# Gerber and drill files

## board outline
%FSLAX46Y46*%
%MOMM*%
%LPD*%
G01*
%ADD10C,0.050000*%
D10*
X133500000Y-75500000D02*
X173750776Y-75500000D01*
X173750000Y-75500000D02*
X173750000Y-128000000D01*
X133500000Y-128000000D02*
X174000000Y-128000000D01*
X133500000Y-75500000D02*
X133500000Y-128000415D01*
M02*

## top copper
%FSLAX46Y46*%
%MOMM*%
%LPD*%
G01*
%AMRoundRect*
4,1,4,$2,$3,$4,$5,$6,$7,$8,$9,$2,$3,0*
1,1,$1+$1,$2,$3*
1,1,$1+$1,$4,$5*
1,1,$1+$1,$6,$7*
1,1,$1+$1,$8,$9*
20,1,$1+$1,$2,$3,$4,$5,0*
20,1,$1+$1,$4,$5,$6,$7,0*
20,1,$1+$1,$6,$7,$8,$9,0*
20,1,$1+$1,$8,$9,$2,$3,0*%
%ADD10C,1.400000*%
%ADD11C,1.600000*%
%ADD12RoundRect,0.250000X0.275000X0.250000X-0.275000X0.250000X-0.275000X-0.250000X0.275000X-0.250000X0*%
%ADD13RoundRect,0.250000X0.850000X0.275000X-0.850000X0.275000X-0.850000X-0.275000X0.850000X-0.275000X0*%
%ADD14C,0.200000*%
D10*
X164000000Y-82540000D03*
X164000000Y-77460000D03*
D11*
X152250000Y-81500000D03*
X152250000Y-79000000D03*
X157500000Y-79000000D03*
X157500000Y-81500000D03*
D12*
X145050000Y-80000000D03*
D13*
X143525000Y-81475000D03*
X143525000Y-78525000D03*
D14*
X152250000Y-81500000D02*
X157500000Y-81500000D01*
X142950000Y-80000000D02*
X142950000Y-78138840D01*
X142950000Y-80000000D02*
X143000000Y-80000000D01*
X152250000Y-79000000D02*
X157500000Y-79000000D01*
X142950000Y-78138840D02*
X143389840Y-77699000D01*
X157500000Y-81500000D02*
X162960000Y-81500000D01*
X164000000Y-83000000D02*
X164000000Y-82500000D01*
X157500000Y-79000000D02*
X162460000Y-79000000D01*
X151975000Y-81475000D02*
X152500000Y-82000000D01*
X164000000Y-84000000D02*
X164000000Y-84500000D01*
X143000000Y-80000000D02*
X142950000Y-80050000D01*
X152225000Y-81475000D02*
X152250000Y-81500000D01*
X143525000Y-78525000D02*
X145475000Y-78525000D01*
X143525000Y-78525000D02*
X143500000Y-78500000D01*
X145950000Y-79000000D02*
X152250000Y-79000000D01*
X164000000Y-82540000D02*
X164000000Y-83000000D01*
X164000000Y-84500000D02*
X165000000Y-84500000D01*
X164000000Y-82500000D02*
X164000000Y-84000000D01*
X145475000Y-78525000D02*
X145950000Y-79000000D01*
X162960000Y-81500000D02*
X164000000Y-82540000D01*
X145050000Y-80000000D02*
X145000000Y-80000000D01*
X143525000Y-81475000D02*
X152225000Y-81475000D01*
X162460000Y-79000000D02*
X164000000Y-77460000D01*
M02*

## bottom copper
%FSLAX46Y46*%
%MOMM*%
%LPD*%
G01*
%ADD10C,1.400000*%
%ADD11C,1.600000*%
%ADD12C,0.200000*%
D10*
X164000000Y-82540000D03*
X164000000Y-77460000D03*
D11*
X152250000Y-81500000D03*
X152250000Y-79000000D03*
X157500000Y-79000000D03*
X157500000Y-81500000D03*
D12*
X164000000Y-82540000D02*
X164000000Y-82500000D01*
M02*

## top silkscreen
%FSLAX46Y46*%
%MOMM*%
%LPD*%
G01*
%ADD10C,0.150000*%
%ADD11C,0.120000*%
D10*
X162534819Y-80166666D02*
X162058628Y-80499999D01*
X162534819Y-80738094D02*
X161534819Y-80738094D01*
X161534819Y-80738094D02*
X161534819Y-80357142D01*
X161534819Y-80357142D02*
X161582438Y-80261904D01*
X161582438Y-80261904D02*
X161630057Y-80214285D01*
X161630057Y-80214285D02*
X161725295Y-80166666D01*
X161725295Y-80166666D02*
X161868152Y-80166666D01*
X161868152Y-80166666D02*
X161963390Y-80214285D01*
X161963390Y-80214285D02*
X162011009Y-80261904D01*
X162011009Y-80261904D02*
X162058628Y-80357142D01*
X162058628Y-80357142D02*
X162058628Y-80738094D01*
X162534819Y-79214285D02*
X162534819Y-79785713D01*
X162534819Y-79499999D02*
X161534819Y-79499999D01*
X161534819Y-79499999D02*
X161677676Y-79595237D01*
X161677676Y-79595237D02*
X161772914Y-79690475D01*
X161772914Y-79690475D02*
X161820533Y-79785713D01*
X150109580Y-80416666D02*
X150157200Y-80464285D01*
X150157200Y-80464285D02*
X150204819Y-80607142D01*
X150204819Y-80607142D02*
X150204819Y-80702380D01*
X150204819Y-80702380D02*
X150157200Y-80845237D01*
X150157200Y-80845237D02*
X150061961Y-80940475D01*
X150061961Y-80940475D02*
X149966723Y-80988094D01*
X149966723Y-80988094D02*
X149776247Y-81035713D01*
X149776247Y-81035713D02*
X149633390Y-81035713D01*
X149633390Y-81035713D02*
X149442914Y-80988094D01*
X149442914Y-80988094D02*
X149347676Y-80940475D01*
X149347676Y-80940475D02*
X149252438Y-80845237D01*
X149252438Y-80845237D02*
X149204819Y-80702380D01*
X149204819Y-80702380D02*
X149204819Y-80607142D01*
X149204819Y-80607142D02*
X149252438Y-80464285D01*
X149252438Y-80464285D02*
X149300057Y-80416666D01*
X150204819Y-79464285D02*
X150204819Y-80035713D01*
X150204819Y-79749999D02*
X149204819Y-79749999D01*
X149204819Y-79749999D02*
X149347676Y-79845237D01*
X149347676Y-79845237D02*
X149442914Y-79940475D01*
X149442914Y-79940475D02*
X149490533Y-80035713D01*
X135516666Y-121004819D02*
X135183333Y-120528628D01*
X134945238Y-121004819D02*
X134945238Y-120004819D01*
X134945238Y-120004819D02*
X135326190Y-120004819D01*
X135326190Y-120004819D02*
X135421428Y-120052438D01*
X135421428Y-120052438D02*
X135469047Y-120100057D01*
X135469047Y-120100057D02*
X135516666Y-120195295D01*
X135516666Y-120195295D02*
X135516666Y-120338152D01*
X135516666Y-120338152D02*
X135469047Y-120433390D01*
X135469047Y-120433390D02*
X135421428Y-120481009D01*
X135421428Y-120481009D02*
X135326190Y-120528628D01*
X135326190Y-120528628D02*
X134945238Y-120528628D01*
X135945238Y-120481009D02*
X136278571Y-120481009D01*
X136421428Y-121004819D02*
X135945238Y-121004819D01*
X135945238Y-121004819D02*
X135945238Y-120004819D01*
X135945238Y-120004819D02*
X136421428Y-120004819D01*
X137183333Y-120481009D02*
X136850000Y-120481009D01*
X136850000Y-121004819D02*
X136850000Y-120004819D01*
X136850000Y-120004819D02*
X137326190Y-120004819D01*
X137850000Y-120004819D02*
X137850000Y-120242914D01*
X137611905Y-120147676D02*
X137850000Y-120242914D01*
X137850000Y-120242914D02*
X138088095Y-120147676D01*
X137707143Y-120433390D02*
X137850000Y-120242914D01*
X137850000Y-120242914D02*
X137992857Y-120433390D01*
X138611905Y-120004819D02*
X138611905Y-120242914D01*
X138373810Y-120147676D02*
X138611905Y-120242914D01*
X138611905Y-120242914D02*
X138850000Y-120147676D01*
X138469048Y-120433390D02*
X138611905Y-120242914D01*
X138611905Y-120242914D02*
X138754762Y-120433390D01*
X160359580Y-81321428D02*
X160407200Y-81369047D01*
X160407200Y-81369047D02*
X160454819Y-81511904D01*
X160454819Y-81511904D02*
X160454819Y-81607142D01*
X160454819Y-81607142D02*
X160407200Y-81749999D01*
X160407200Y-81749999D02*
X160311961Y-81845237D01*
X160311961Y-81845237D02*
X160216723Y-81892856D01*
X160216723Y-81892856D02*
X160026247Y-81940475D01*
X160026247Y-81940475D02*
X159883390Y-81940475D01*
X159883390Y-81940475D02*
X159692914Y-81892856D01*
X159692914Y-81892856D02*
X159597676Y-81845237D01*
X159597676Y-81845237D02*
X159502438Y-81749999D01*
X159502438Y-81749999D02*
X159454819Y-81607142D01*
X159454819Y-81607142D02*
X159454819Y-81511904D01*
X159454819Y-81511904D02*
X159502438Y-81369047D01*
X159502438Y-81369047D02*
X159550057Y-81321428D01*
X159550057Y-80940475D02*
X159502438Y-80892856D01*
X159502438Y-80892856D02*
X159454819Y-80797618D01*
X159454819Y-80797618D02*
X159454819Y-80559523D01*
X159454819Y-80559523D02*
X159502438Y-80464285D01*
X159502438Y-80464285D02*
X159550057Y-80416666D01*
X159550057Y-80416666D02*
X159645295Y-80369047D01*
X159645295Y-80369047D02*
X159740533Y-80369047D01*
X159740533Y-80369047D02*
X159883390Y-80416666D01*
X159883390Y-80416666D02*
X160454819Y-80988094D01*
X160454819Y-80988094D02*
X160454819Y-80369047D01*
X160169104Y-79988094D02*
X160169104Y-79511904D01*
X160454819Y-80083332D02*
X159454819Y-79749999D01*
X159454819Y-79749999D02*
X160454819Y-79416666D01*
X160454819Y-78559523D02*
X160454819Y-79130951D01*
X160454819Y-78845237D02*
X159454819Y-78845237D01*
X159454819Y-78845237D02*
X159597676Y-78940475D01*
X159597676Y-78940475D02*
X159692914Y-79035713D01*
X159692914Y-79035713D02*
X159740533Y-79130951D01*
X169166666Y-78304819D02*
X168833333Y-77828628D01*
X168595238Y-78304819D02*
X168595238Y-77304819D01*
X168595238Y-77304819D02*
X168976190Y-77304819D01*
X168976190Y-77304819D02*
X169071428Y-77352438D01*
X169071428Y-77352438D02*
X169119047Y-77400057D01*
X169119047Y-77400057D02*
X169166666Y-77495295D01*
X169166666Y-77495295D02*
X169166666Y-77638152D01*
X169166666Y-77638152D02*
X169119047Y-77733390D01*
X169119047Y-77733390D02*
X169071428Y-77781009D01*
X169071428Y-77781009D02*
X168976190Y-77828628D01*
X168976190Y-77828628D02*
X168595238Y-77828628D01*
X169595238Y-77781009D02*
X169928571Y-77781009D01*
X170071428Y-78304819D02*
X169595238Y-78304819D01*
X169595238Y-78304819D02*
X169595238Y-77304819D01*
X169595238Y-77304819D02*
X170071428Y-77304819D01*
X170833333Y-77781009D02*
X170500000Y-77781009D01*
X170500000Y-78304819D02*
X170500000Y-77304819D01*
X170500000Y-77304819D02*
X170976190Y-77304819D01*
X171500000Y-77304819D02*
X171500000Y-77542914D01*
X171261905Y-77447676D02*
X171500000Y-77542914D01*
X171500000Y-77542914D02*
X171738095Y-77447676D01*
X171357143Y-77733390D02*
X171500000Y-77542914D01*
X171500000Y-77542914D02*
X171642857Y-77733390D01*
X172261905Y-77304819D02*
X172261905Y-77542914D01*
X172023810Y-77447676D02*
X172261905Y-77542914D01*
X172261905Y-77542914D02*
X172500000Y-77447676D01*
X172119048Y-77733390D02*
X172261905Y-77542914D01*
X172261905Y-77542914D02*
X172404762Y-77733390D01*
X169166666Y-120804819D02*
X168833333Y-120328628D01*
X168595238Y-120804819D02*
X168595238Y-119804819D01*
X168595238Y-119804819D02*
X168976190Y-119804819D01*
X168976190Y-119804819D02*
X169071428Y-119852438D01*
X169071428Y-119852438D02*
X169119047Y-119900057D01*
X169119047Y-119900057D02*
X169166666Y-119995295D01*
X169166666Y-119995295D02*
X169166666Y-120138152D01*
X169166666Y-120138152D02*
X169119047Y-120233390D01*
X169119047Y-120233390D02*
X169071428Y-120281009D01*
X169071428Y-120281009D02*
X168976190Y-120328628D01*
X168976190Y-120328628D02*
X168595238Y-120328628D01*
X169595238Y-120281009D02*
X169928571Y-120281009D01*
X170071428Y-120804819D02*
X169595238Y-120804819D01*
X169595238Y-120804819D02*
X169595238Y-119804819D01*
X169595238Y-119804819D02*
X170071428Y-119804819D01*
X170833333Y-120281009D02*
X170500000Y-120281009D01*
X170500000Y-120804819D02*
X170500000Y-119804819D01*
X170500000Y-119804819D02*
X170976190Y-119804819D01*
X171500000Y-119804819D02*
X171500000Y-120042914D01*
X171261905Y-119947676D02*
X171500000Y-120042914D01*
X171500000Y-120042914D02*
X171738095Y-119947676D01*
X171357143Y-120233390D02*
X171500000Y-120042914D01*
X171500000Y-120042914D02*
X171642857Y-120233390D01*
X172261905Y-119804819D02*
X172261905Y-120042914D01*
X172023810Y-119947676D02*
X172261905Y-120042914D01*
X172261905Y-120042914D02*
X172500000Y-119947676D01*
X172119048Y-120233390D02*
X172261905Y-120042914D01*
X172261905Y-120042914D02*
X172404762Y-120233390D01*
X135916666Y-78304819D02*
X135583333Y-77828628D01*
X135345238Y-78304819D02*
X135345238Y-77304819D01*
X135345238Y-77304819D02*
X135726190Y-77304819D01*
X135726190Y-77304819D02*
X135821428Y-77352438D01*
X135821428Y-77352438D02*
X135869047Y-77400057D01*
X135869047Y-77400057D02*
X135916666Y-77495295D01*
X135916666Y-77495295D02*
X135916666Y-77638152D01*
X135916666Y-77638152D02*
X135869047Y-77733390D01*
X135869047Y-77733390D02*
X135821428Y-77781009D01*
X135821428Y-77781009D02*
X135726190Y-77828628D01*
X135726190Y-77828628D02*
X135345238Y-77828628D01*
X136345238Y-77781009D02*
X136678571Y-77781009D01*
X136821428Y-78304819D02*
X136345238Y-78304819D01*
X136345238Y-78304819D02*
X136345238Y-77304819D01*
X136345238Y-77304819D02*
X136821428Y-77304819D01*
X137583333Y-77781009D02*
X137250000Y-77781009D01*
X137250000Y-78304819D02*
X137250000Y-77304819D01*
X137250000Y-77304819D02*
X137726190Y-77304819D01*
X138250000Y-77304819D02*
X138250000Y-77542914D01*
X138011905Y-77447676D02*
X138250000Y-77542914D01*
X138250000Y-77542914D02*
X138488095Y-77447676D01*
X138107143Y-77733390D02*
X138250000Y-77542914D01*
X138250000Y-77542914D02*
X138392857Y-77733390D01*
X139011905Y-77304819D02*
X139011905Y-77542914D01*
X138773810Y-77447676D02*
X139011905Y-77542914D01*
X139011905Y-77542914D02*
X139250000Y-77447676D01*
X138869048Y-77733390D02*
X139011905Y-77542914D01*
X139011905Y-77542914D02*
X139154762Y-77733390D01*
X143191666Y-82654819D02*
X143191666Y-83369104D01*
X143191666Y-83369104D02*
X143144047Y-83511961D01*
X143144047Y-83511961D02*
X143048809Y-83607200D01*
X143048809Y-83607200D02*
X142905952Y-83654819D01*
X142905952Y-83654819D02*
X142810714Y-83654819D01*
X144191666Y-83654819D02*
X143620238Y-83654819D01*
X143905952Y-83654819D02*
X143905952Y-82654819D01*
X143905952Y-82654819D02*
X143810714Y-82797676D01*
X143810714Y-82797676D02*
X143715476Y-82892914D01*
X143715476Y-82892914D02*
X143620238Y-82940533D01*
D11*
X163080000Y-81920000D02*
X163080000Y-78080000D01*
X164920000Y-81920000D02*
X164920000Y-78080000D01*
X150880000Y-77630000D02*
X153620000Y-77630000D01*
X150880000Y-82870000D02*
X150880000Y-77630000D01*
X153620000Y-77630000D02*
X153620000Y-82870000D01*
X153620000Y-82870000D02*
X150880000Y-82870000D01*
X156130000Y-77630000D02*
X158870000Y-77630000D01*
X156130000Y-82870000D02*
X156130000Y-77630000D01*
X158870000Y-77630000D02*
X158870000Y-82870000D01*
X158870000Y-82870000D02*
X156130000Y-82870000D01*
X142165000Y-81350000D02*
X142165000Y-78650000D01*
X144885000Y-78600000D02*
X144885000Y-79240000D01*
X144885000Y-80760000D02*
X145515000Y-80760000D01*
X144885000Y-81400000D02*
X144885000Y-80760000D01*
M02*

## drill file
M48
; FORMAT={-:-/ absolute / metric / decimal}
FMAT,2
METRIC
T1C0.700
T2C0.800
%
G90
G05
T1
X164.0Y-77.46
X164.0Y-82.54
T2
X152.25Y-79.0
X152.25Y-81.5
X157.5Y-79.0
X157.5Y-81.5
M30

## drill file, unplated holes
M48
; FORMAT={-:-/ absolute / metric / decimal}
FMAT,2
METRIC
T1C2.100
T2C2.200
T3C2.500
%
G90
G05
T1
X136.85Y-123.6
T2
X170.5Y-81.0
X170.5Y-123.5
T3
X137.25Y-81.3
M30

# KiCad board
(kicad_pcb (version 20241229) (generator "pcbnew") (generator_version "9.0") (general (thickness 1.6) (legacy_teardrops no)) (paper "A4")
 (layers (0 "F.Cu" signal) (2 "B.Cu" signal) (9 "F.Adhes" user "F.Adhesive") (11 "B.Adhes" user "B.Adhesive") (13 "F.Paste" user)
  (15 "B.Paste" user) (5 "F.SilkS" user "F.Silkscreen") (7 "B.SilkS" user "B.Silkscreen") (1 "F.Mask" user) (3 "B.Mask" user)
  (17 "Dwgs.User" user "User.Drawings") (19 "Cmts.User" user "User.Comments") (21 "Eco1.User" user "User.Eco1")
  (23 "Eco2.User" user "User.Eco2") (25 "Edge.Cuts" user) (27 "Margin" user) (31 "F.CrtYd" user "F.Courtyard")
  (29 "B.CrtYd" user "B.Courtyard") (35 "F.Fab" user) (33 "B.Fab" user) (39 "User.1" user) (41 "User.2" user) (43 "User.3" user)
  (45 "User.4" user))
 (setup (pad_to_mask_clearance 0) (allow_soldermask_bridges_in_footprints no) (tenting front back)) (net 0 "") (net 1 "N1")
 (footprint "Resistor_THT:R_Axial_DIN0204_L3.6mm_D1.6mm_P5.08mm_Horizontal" (layer "F.Cu") (at 164 82.54 90)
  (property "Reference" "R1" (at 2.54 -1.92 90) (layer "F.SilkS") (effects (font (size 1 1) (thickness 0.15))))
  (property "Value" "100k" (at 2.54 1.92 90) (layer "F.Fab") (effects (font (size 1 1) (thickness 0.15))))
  (fp_line (start 0.62 -0.92) (end 4.46 -0.92) (stroke (width 0.12) (type solid)) (layer "F.SilkS"))
  (fp_line (start 0.62 0.92) (end 4.46 0.92) (stroke (width 0.12) (type solid)) (layer "F.SilkS"))
  (pad "1" thru_hole circle (at 0 0 90) (size 1.4 1.4) (drill 0.7) (layers "*.Cu" "*.Mask") (remove_unused_layers no) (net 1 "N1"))
  (pad "2" thru_hole circle (at 5.08 0 90) (size 1.4 1.4) (drill 0.7) (layers "*.Cu" "*.Mask") (remove_unused_layers no) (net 1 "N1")))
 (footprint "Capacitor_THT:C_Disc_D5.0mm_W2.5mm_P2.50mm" (layer "F.Cu") (at 152.25 81.5 90)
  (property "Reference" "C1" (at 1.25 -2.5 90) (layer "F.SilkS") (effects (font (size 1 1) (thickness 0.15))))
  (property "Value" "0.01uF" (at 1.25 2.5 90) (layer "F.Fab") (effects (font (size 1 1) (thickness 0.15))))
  (fp_line (start 3.87 -1.37) (end 3.87 1.37) (stroke (width 0.12) (type solid)) (layer "F.SilkS"))
  (fp_line (start -1.37 -1.37) (end 3.87 -1.37) (stroke (width 0.12) (type solid)) (layer "F.SilkS"))
  (fp_line (start 3.87 1.37) (end -1.37 1.37) (stroke (width 0.12) (type solid)) (layer "F.SilkS"))
  (fp_line (start -1.37 1.37) (end -1.37 -1.37) (stroke (width 0.12) (type solid)) (layer "F.SilkS"))
  (pad "1" thru_hole circle (at 0 0 90) (size 1.6 1.6) (drill 0.8) (layers "*.Cu" "*.Mask") (remove_unused_layers no) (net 1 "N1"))
  (pad "2" thru_hole circle (at 2.5 0 90) (size 1.6 1.6) (drill 0.8) (layers "*.Cu" "*.Mask") (remove_unused_layers no) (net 1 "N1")))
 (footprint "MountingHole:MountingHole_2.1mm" (layer "F.Cu") (at 136.85 123.6)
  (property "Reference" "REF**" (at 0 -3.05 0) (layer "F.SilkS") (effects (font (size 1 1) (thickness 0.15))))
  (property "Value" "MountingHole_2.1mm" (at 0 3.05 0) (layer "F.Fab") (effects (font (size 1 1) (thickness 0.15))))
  (pad "" np_thru_hole circle (at 0 0) (size 2.1 2.1) (drill 2.1) (layers "*.Cu" "*.Mask")))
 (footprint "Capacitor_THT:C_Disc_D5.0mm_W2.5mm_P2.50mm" (layer "F.Cu") (at 157.5 79 -90)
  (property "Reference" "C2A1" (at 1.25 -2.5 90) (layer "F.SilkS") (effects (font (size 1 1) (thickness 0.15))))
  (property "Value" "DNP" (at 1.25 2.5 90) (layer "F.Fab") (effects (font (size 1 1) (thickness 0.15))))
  (fp_line (start -1.37 1.37) (end -1.37 -1.37) (stroke (width 0.12) (type solid)) (layer "F.SilkS"))
  (fp_line (start 3.87 1.37) (end -1.37 1.37) (stroke (width 0.12) (type solid)) (layer "F.SilkS"))
  (fp_line (start -1.37 -1.37) (end 3.87 -1.37) (stroke (width 0.12) (type solid)) (layer "F.SilkS"))
  (fp_line (start 3.87 -1.37) (end 3.87 1.37) (stroke (width 0.12) (type solid)) (layer "F.SilkS"))
  (pad "1" thru_hole circle (at 0 0 270) (size 1.6 1.6) (drill 0.8) (layers "*.Cu" "*.Mask") (remove_unused_layers no) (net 1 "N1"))
  (pad "2" thru_hole circle (at 2.5 0 270) (size 1.6 1.6) (drill 0.8) (layers "*.Cu" "*.Mask") (remove_unused_layers no) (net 1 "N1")))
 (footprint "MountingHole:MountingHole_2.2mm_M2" (layer "F.Cu") (at 170.5 81)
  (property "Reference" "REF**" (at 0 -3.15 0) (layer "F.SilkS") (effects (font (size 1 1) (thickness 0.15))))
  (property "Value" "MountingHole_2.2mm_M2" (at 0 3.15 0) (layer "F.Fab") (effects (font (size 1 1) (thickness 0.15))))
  (pad "" np_thru_hole circle (at 0 0) (size 2.2 2.2) (drill 2.2) (layers "*.Cu" "*.Mask")))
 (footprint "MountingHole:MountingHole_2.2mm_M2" (layer "F.Cu") (at 170.5 123.5)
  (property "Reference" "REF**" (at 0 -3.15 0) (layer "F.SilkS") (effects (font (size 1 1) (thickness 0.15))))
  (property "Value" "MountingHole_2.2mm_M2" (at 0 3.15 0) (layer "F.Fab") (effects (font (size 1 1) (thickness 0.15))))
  (pad "" np_thru_hole circle (at 0 0) (size 2.2 2.2) (drill 2.2) (layers "*.Cu" "*.Mask")))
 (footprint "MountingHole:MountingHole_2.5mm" (layer "F.Cu") (at 137.25 81.3)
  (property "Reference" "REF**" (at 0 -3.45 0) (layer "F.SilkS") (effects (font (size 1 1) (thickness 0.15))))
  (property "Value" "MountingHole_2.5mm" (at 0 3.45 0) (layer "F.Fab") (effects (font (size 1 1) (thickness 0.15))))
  (pad "" np_thru_hole circle (at 0 0) (size 2.5 2.5) (drill 2.5) (layers "*.Cu" "*.Mask")))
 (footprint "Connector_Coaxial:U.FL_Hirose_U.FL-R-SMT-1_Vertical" (layer "F.Cu") (at 144 80 180)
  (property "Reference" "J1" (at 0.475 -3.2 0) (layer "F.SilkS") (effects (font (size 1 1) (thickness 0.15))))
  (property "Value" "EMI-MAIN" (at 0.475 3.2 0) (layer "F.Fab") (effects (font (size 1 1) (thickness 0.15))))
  (fp_line (start 1.835 -1.35) (end 1.835 1.35) (stroke (width 0.12) (type solid)) (layer "F.SilkS"))
  (fp_line (start -0.885 1.4) (end -0.885 0.76) (stroke (width 0.12) (type solid)) (layer "F.SilkS"))
  (fp_line (start -0.885 -0.76) (end -1.515 -0.76) (stroke (width 0.12) (type solid)) (layer "F.SilkS"))
  (fp_line (start -0.885 -1.4) (end -0.885 -0.76) (stroke (width 0.12) (type solid)) (layer "F.SilkS"))
  (pad "1" smd roundrect (at -1.05 0 180) (size 1.05 1) (layers "F.Cu" "F.Mask" "F.Paste") (roundrect_rratio 0.25) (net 1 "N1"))
  (pad "2" smd roundrect (at 0.475 -1.475 180) (size 2.2 1.05) (layers "F.Cu" "F.Mask" "F.Paste") (roundrect_rratio 0.2380952381)
   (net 1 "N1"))
  (pad "2" smd roundrect (at 0.475 1.475 180) (size 2.2 1.05) (layers "F.Cu" "F.Mask" "F.Paste") (roundrect_rratio 0.2380952381)
   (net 1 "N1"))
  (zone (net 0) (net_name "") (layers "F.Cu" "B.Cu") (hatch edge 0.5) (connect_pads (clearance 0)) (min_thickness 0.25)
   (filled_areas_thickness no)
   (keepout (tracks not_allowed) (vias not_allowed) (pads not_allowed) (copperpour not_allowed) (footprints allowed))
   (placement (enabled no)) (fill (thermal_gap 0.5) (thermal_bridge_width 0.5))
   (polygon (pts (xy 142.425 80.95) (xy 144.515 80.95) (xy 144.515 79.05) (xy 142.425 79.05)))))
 (gr_line (start 133.5 75.5) (end 173.750776 75.5) (stroke (width 0.05) (type solid)) (layer "Edge.Cuts"))
 (gr_line (start 173.75 75.5) (end 173.75 128) (stroke (width 0.05) (type default)) (layer "Edge.Cuts"))
 (gr_line (start 133.5 128) (end 174 128) (stroke (width 0.05) (type default)) (layer "Edge.Cuts"))
 (gr_line (start 133.5 75.5) (end 133.5 128.000415) (stroke (width 0.05) (type solid)) (layer "Edge.Cuts"))
 (segment (start 152.25 81.5) (end 157.5 81.5) (width 0.2) (layer "F.Cu") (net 1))
 (segment (start 142.95 80) (end 142.95 78.13884) (width 0.2) (layer "F.Cu") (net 1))
 (segment (start 142.95 80) (end 143 80) (width 0.2) (layer "F.Cu") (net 1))
 (segment (start 152.25 79) (end 157.5 79) (width 0.2) (layer "F.Cu") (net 1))
 (segment (start 142.95 78.13884) (end 143.38984 77.699) (width 0.2) (layer "F.Cu") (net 1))
 (segment (start 157.5 81.5) (end 162.96 81.5) (width 0.2) (layer "F.Cu") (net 1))
 (segment (start 164 83) (end 164 82.5) (width 0.2) (layer "F.Cu") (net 1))
 (segment (start 157.5 79) (end 162.46 79) (width 0.2) (layer "F.Cu") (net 1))
 (segment (start 151.975 81.475) (end 152.5 82) (width 0.2) (layer "F.Cu") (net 1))
 (segment (start 164 84) (end 164 84.5) (width 0.2) (layer "F.Cu") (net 1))
 (segment (start 143 80) (end 142.95 80.05) (width 0.2) (layer "F.Cu") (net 1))
 (segment (start 152.225 81.475) (end 152.25 81.5) (width 0.2) (layer "F.Cu") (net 1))
 (segment (start 143.525 78.525) (end 145.475 78.525) (width 0.2) (layer "F.Cu") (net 1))
 (segment (start 143.525 78.525) (end 143.5 78.5) (width 0.2) (layer "F.Cu") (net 1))
 (segment (start 145.95 79) (end 152.25 79) (width 0.2) (layer "F.Cu") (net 1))
 (segment (start 164 82.54) (end 164 83) (width 0.2) (layer "F.Cu") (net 1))
 (segment (start 164 84.5) (end 165 84.5) (width 0.2) (layer "F.Cu") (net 1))
 (segment (start 164 82.5) (end 164 84) (width 0.2) (layer "F.Cu") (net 1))
 (segment (start 145.475 78.525) (end 145.95 79) (width 0.2) (layer "F.Cu") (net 1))
 (segment (start 162.96 81.5) (end 164 82.54) (width 0.2) (layer "F.Cu") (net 1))
 (segment (start 145.05 80) (end 145 80) (width 0.2) (layer "F.Cu") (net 1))
 (segment (start 143.525 81.475) (end 152.225 81.475) (width 0.2) (layer "F.Cu") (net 1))
 (segment (start 162.46 79) (end 164 77.46) (width 0.2) (layer "F.Cu") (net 1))
 (segment (start 164 82.54) (end 164 82.5) (width 0.2) (layer "B.Cu") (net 1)))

